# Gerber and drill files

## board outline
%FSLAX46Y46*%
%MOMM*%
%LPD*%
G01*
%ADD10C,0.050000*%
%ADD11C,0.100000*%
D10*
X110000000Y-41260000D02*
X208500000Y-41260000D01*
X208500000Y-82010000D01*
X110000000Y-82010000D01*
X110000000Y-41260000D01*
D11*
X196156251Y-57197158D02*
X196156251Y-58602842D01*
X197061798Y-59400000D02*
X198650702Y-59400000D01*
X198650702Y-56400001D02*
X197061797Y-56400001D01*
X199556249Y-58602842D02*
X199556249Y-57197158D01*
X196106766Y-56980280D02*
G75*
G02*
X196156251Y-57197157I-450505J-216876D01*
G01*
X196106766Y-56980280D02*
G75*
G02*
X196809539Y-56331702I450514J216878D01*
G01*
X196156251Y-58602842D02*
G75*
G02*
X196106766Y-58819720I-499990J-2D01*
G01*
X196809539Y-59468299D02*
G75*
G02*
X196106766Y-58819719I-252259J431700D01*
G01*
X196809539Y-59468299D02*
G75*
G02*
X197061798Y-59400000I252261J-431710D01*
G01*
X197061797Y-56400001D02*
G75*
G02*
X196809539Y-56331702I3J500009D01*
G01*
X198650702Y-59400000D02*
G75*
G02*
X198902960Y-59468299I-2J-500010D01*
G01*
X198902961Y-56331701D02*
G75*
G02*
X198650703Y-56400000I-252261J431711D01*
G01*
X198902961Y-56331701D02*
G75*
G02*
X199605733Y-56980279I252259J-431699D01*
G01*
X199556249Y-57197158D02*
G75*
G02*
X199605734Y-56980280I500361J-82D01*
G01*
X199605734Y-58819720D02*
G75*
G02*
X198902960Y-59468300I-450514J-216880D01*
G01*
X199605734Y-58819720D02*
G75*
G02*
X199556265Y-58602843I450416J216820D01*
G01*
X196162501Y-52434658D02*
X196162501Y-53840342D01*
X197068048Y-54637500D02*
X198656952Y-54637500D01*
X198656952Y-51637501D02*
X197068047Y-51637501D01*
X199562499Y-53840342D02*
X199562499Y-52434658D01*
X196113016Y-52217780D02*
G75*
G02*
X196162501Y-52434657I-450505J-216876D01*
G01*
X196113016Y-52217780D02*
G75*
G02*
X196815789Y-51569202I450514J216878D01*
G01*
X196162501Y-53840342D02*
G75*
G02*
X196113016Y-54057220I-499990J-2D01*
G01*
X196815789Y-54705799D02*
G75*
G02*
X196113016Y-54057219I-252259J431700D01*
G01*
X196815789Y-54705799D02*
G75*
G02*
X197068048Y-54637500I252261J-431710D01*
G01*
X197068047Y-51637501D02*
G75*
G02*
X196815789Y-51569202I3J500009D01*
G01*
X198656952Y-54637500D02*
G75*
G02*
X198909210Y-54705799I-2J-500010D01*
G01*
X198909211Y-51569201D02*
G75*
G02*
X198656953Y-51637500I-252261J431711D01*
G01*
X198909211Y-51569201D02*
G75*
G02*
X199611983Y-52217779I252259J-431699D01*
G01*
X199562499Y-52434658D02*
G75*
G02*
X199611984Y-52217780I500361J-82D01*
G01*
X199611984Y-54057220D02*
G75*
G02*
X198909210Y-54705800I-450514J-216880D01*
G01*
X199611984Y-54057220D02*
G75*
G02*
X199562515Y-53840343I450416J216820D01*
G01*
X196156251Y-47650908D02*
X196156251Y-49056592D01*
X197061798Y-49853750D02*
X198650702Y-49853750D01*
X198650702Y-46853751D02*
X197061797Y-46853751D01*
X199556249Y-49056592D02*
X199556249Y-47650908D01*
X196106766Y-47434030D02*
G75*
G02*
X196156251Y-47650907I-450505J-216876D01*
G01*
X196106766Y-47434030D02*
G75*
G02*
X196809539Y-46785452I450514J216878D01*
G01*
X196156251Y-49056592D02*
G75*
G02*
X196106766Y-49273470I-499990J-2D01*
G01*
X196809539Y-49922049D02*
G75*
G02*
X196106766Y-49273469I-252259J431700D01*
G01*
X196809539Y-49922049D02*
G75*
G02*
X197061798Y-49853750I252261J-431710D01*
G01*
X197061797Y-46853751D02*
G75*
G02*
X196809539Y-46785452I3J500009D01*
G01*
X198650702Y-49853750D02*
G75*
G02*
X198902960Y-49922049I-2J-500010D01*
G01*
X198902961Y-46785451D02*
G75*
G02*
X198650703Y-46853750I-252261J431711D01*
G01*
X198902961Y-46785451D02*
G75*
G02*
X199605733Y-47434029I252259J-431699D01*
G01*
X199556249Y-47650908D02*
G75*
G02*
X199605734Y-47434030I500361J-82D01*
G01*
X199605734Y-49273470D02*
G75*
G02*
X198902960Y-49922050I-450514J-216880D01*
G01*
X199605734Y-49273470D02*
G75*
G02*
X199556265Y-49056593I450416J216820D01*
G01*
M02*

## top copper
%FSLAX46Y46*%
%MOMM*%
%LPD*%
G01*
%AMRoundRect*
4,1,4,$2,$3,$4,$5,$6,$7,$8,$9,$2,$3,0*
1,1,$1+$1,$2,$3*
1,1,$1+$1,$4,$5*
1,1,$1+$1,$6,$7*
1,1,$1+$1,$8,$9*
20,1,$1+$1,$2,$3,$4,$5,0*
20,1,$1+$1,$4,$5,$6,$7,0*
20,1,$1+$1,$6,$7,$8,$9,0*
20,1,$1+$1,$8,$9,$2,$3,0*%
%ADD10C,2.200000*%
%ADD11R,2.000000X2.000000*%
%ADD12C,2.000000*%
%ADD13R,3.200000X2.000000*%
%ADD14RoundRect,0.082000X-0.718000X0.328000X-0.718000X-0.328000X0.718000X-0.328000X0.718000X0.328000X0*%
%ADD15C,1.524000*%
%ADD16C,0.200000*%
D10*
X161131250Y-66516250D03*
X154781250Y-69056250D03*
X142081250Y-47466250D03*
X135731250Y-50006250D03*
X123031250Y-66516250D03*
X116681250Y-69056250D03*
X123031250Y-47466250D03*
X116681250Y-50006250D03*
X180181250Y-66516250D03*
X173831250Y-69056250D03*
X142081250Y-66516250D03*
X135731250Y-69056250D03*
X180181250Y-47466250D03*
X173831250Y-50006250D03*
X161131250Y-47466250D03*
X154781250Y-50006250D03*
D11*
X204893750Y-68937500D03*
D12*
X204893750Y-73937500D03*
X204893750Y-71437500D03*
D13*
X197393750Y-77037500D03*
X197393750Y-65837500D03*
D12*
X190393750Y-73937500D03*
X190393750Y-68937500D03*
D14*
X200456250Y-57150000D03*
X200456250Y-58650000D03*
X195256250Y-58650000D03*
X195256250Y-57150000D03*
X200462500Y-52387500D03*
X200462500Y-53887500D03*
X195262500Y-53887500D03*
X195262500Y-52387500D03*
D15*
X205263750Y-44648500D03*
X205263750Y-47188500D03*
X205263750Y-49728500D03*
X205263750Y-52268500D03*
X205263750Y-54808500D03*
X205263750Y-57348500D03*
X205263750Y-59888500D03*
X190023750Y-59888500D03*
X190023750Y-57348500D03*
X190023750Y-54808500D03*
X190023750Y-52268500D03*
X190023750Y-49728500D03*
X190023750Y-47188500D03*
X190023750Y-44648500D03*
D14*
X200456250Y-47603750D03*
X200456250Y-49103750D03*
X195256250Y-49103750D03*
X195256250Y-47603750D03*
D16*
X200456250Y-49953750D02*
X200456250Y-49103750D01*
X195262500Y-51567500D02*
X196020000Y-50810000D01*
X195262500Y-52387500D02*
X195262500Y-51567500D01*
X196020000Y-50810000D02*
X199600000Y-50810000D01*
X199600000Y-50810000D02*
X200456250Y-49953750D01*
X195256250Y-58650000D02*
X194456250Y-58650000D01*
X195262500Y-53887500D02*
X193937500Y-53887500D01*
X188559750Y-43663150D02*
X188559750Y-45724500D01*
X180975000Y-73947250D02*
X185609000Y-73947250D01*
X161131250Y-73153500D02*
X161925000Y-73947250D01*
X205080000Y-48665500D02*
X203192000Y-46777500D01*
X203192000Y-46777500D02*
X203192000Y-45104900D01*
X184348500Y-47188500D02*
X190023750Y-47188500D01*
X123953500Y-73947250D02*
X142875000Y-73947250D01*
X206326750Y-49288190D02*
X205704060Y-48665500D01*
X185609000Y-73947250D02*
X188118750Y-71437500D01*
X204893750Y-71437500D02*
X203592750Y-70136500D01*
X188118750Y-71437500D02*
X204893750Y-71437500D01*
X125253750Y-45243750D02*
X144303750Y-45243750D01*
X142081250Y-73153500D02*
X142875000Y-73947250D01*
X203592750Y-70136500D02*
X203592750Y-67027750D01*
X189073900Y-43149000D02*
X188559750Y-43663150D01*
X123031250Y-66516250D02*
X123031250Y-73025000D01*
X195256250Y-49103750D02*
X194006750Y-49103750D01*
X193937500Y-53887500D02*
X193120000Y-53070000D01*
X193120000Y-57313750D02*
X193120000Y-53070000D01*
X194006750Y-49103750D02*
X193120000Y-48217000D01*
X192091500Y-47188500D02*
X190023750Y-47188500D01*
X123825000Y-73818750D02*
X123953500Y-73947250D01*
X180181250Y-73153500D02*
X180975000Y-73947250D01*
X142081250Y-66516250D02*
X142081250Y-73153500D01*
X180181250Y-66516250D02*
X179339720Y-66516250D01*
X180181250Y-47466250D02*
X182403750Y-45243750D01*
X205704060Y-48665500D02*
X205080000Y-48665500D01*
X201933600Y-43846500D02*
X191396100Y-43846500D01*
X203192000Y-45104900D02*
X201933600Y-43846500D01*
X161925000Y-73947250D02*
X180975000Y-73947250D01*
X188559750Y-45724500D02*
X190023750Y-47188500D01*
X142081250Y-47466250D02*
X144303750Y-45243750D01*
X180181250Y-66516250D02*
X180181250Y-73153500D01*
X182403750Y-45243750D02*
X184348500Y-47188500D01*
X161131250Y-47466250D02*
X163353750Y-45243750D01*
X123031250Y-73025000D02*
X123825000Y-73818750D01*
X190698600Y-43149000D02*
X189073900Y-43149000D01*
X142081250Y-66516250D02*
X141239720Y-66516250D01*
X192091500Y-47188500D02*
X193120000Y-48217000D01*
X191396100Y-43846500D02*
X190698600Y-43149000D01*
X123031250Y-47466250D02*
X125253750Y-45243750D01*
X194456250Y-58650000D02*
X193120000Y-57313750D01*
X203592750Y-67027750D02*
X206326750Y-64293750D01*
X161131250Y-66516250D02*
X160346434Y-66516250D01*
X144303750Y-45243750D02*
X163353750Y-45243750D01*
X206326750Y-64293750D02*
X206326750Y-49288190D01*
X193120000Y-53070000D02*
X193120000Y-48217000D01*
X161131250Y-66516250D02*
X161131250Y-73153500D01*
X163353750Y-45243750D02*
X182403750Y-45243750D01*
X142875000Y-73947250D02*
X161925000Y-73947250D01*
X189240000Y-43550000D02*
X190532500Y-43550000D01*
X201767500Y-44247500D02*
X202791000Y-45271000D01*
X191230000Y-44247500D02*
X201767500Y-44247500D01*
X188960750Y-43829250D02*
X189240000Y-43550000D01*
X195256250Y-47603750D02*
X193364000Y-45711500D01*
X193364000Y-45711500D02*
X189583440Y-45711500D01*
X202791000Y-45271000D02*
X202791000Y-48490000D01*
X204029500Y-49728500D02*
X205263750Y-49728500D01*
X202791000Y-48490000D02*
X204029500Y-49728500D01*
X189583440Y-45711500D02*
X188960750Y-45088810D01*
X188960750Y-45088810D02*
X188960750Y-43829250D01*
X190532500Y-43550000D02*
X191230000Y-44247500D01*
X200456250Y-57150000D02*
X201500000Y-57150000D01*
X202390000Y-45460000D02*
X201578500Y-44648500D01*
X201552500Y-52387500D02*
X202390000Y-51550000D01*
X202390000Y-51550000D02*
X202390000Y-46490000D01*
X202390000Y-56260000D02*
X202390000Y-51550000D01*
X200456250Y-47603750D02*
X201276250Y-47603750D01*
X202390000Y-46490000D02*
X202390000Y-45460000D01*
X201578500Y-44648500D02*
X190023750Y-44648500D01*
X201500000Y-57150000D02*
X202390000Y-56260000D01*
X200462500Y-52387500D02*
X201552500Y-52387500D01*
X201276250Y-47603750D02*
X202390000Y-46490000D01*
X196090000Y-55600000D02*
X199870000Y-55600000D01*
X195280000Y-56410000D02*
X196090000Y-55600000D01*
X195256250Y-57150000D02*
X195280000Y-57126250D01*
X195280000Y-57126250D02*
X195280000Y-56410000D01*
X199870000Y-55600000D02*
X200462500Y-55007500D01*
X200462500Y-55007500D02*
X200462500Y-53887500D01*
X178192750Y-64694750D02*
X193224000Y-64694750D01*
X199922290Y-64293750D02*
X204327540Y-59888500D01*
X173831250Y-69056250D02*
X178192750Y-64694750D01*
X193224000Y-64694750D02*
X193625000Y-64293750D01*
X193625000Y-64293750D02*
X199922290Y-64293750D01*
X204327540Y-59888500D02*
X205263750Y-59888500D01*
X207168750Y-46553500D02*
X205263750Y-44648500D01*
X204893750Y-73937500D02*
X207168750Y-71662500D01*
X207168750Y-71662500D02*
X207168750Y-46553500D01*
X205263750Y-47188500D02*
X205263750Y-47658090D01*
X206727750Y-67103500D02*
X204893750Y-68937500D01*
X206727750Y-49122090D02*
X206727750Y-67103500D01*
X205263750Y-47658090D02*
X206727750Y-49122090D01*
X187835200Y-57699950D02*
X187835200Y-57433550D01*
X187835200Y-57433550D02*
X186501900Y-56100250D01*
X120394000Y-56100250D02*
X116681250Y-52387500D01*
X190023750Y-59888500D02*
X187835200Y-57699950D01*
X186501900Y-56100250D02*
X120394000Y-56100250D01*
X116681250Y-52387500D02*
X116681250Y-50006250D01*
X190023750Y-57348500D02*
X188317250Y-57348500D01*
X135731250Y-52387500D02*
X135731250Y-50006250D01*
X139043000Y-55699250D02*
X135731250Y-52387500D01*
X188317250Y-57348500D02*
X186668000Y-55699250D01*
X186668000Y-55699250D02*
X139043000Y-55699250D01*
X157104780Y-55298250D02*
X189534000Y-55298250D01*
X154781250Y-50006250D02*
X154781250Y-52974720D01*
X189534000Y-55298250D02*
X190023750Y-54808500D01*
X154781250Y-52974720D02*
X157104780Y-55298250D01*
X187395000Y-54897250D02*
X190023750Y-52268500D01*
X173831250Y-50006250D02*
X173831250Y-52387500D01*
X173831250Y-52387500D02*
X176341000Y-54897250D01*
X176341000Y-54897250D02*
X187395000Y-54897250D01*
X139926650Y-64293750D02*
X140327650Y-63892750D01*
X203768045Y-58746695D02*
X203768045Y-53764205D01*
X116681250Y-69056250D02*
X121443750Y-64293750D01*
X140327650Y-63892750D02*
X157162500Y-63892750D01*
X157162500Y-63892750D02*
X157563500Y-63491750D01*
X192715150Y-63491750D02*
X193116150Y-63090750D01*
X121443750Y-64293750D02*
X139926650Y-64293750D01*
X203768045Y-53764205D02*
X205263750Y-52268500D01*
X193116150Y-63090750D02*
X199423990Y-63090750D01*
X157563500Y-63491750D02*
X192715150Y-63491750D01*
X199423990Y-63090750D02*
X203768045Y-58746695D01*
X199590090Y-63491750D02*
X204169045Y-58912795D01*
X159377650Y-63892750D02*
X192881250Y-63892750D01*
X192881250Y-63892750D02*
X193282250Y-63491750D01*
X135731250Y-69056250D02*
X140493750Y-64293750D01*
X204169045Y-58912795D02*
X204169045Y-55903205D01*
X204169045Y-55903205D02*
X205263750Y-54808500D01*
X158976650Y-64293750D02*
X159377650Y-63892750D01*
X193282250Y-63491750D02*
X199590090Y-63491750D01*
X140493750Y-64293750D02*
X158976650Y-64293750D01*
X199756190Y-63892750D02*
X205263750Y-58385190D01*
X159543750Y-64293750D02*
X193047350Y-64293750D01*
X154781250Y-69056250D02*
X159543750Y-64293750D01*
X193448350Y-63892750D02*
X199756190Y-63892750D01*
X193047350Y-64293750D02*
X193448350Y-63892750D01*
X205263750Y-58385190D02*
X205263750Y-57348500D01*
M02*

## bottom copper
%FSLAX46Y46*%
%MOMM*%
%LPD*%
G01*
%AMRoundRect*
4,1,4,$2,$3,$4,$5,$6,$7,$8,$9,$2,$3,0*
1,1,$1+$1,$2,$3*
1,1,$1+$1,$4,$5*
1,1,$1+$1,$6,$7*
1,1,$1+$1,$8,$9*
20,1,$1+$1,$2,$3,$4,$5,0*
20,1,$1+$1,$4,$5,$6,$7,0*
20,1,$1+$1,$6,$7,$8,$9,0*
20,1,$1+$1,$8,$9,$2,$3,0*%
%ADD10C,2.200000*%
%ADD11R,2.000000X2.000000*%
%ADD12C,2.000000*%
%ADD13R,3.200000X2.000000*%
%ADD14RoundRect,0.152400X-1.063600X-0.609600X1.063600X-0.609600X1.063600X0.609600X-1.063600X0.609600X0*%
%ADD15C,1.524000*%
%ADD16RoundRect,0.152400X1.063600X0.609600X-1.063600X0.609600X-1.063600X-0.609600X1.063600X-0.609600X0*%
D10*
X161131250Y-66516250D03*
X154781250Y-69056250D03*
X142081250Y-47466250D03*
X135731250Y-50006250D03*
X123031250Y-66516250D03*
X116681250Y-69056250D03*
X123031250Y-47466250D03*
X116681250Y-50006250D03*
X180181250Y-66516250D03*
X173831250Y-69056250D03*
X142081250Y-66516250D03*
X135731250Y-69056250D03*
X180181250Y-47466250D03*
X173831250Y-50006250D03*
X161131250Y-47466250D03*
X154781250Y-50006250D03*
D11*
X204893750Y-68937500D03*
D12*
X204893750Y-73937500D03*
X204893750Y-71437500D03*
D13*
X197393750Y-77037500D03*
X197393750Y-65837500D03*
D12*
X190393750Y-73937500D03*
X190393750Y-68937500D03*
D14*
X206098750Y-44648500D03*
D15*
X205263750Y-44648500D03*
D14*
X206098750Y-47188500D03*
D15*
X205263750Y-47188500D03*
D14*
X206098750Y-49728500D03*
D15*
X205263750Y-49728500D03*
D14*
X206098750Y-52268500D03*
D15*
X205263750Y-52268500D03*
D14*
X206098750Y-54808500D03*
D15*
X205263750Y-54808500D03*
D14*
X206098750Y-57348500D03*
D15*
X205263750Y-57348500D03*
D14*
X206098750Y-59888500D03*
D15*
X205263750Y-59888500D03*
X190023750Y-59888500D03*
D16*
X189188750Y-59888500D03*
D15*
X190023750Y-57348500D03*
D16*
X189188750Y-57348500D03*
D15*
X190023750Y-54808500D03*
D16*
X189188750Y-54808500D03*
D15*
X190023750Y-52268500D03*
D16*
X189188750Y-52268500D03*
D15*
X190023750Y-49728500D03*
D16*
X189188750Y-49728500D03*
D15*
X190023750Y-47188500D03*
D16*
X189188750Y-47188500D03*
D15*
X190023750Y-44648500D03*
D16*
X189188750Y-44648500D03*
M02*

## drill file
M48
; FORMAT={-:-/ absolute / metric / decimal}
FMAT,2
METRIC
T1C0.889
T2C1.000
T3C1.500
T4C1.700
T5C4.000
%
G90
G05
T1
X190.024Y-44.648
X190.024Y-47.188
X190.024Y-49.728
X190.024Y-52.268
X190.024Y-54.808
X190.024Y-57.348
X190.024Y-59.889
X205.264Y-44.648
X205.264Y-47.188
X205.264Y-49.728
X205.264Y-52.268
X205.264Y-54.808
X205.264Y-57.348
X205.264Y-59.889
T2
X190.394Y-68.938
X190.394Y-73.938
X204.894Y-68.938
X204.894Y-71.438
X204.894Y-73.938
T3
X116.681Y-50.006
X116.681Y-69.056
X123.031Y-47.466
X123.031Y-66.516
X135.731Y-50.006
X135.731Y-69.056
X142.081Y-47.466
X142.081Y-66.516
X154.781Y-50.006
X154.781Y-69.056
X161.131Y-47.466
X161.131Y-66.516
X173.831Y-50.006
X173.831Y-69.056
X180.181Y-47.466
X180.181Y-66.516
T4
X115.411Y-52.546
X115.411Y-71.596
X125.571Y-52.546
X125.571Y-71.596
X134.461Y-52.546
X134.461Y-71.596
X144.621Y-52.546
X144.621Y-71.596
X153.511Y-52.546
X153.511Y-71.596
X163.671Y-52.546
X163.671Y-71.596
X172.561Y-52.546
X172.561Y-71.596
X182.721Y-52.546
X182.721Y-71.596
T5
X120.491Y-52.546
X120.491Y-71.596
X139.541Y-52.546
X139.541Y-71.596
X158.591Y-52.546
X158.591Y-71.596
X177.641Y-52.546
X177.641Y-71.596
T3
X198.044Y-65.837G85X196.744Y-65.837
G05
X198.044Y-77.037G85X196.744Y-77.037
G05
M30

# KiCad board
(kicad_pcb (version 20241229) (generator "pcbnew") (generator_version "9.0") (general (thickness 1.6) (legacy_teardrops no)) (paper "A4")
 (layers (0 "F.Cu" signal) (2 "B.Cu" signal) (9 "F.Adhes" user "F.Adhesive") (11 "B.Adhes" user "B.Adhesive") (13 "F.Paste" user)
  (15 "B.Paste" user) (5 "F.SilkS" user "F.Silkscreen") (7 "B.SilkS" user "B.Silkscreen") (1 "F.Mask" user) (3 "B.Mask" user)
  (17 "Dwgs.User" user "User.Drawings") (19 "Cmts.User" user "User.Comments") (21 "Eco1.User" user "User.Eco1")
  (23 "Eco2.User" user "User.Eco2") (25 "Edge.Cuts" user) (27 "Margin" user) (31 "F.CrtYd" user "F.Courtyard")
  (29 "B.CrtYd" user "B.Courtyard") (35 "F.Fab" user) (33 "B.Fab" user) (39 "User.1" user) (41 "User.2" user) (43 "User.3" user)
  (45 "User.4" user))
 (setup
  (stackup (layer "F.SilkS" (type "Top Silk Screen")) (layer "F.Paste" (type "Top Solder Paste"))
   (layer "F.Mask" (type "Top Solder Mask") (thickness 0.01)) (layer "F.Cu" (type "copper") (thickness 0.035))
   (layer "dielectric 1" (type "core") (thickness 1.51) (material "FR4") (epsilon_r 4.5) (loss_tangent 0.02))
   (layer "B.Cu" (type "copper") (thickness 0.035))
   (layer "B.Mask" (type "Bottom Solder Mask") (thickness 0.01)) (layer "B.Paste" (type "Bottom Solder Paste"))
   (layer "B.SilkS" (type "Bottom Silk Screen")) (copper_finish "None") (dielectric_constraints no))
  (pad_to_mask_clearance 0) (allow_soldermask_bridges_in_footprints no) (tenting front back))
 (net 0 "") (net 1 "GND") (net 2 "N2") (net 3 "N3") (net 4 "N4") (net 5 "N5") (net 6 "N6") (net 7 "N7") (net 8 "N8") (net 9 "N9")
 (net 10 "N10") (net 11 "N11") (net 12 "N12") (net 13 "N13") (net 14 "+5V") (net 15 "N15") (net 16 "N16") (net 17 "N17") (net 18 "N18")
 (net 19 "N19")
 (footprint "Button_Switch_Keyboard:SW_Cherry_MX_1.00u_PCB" (layer "F.Cu") (at 161.13125 66.51625)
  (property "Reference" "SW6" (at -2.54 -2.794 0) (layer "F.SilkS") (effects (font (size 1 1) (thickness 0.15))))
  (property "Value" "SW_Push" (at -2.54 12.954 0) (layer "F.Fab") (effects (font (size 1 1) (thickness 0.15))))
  (pad "" np_thru_hole circle (at -7.62 5.08) (size 1.7 1.7) (drill 1.7) (layers "*.Cu" "*.Mask"))
  (pad "" np_thru_hole circle (at -2.54 5.08) (size 4 4) (drill 4) (layers "*.Cu" "*.Mask"))
  (pad "" np_thru_hole circle (at 2.54 5.08) (size 1.7 1.7) (drill 1.7) (layers "*.Cu" "*.Mask"))
  (pad "1" thru_hole circle (at 0 0) (size 2.2 2.2) (drill 1.5) (layers "*.Cu" "*.Mask") (remove_unused_layers no) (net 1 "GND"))
  (pad "2" thru_hole circle (at -6.35 2.54) (size 2.2 2.2) (drill 1.5) (layers "*.Cu" "*.Mask") (remove_unused_layers no) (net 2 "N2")))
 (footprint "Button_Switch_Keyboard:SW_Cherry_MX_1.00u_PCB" (layer "F.Cu") (at 142.08125 47.46625)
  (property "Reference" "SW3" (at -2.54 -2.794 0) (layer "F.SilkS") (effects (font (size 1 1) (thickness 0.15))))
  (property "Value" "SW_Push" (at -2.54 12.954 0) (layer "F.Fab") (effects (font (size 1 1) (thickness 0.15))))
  (pad "" np_thru_hole circle (at -7.62 5.08) (size 1.7 1.7) (drill 1.7) (layers "*.Cu" "*.Mask"))
  (pad "" np_thru_hole circle (at -2.54 5.08) (size 4 4) (drill 4) (layers "*.Cu" "*.Mask"))
  (pad "" np_thru_hole circle (at 2.54 5.08) (size 1.7 1.7) (drill 1.7) (layers "*.Cu" "*.Mask"))
  (pad "1" thru_hole circle (at 0 0) (size 2.2 2.2) (drill 1.5) (layers "*.Cu" "*.Mask") (remove_unused_layers no) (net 1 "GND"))
  (pad "2" thru_hole circle (at -6.35 2.54) (size 2.2 2.2) (drill 1.5) (layers "*.Cu" "*.Mask") (remove_unused_layers no) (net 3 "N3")))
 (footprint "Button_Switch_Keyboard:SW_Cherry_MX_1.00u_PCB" (layer "F.Cu") (at 123.03125 66.51625)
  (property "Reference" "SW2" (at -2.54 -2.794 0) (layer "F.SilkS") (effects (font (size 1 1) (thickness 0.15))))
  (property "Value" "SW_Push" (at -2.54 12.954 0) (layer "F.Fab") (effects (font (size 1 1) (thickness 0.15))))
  (pad "" np_thru_hole circle (at -7.62 5.08) (size 1.7 1.7) (drill 1.7) (layers "*.Cu" "*.Mask"))
  (pad "" np_thru_hole circle (at -2.54 5.08) (size 4 4) (drill 4) (layers "*.Cu" "*.Mask"))
  (pad "" np_thru_hole circle (at 2.54 5.08) (size 1.7 1.7) (drill 1.7) (layers "*.Cu" "*.Mask"))
  (pad "1" thru_hole circle (at 0 0) (size 2.2 2.2) (drill 1.5) (layers "*.Cu" "*.Mask") (remove_unused_layers no) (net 1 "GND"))
  (pad "2" thru_hole circle (at -6.35 2.54) (size 2.2 2.2) (drill 1.5) (layers "*.Cu" "*.Mask") (remove_unused_layers no) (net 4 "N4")))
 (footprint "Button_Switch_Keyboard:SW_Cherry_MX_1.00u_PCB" (layer "F.Cu") (at 123.03125 47.46625)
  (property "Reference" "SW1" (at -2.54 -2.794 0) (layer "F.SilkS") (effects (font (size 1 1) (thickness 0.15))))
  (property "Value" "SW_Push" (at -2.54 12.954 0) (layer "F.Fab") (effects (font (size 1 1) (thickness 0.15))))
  (pad "" np_thru_hole circle (at -7.62 5.08) (size 1.7 1.7) (drill 1.7) (layers "*.Cu" "*.Mask"))
  (pad "" np_thru_hole circle (at -2.54 5.08) (size 4 4) (drill 4) (layers "*.Cu" "*.Mask"))
  (pad "" np_thru_hole circle (at 2.54 5.08) (size 1.7 1.7) (drill 1.7) (layers "*.Cu" "*.Mask"))
  (pad "1" thru_hole circle (at 0 0) (size 2.2 2.2) (drill 1.5) (layers "*.Cu" "*.Mask") (remove_unused_layers no) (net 1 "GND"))
  (pad "2" thru_hole circle (at -6.35 2.54) (size 2.2 2.2) (drill 1.5) (layers "*.Cu" "*.Mask") (remove_unused_layers no) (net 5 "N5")))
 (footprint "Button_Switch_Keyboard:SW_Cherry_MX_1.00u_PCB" (layer "F.Cu") (at 180.18125 66.51625)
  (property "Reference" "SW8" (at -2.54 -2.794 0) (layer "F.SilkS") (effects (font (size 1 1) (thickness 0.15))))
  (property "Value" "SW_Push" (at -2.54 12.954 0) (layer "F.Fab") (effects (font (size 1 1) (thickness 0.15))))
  (pad "" np_thru_hole circle (at -7.62 5.08) (size 1.7 1.7) (drill 1.7) (layers "*.Cu" "*.Mask"))
  (pad "" np_thru_hole circle (at -2.54 5.08) (size 4 4) (drill 4) (layers "*.Cu" "*.Mask"))
  (pad "" np_thru_hole circle (at 2.54 5.08) (size 1.7 1.7) (drill 1.7) (layers "*.Cu" "*.Mask"))
  (pad "1" thru_hole circle (at 0 0) (size 2.2 2.2) (drill 1.5) (layers "*.Cu" "*.Mask") (remove_unused_layers no) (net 1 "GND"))
  (pad "2" thru_hole circle (at -6.35 2.54) (size 2.2 2.2) (drill 1.5) (layers "*.Cu" "*.Mask") (remove_unused_layers no) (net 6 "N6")))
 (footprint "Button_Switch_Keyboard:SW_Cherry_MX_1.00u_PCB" (layer "F.Cu") (at 142.08125 66.51625)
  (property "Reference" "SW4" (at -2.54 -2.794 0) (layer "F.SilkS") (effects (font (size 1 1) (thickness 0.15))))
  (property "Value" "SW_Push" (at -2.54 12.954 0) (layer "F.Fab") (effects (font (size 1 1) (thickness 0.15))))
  (pad "" np_thru_hole circle (at -7.62 5.08) (size 1.7 1.7) (drill 1.7) (layers "*.Cu" "*.Mask"))
  (pad "" np_thru_hole circle (at -2.54 5.08) (size 4 4) (drill 4) (layers "*.Cu" "*.Mask"))
  (pad "" np_thru_hole circle (at 2.54 5.08) (size 1.7 1.7) (drill 1.7) (layers "*.Cu" "*.Mask"))
  (pad "1" thru_hole circle (at 0 0) (size 2.2 2.2) (drill 1.5) (layers "*.Cu" "*.Mask") (remove_unused_layers no) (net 1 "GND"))
  (pad "2" thru_hole circle (at -6.35 2.54) (size 2.2 2.2) (drill 1.5) (layers "*.Cu" "*.Mask") (remove_unused_layers no) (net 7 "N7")))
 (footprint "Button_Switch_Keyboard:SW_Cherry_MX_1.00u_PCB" (layer "F.Cu") (at 180.18125 47.46625)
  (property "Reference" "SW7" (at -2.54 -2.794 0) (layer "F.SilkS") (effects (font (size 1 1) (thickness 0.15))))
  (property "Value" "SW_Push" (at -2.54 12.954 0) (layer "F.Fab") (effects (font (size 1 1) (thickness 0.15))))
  (pad "" np_thru_hole circle (at -7.62 5.08) (size 1.7 1.7) (drill 1.7) (layers "*.Cu" "*.Mask"))
  (pad "" np_thru_hole circle (at -2.54 5.08) (size 4 4) (drill 4) (layers "*.Cu" "*.Mask"))
  (pad "" np_thru_hole circle (at 2.54 5.08) (size 1.7 1.7) (drill 1.7) (layers "*.Cu" "*.Mask"))
  (pad "1" thru_hole circle (at 0 0) (size 2.2 2.2) (drill 1.5) (layers "*.Cu" "*.Mask") (remove_unused_layers no) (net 1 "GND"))
  (pad "2" thru_hole circle (at -6.35 2.54) (size 2.2 2.2) (drill 1.5) (layers "*.Cu" "*.Mask") (remove_unused_layers no) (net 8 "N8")))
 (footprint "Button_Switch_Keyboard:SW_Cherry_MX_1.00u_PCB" (layer "F.Cu") (at 161.13125 47.46625)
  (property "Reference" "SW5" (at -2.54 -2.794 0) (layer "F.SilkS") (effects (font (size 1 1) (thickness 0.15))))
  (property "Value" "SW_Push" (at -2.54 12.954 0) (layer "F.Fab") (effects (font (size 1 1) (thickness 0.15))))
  (pad "" np_thru_hole circle (at -7.62 5.08) (size 1.7 1.7) (drill 1.7) (layers "*.Cu" "*.Mask"))
  (pad "" np_thru_hole circle (at -2.54 5.08) (size 4 4) (drill 4) (layers "*.Cu" "*.Mask"))
  (pad "" np_thru_hole circle (at 2.54 5.08) (size 1.7 1.7) (drill 1.7) (layers "*.Cu" "*.Mask"))
  (pad "1" thru_hole circle (at 0 0) (size 2.2 2.2) (drill 1.5) (layers "*.Cu" "*.Mask") (remove_unused_layers no) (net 1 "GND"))
  (pad "2" thru_hole circle (at -6.35 2.54) (size 2.2 2.2) (drill 1.5) (layers "*.Cu" "*.Mask") (remove_unused_layers no) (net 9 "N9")))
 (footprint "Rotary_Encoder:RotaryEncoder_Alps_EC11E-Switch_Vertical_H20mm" (layer "B.Cu") (at 204.89375 68.9375 180)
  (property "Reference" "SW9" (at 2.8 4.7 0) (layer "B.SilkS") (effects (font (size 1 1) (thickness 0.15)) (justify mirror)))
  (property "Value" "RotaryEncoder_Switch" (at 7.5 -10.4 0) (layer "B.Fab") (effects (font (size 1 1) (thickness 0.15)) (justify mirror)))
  (pad "A" thru_hole rect (at 0 0 180) (size 2 2) (drill 1) (layers "*.Cu" "*.Mask") (remove_unused_layers no) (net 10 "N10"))
  (pad "B" thru_hole circle (at 0 -5 180) (size 2 2) (drill 1) (layers "*.Cu" "*.Mask") (remove_unused_layers no) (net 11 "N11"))
  (pad "C" thru_hole circle (at 0 -2.5 180) (size 2 2) (drill 1) (layers "*.Cu" "*.Mask") (remove_unused_layers no) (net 1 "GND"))
  (pad "MP" thru_hole rect (at 7.5 -8.1 180) (size 3.2 2) (drill oval 2.8 1.5) (layers "*.Cu" "*.Mask") (remove_unused_layers no))
  (pad "MP" thru_hole rect (at 7.5 3.1 180) (size 3.2 2) (drill oval 2.8 1.5) (layers "*.Cu" "*.Mask") (remove_unused_layers no))
  (pad "S1" thru_hole circle (at 14.5 -5 180) (size 2 2) (drill 1) (layers "*.Cu" "*.Mask") (remove_unused_layers no) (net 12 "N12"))
  (pad "S2" thru_hole circle (at 14.5 0 180) (size 2 2) (drill 1) (layers "*.Cu" "*.Mask") (remove_unused_layers no) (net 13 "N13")))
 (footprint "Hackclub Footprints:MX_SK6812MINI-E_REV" (layer "B.Cu") (at 197.85625 62.98)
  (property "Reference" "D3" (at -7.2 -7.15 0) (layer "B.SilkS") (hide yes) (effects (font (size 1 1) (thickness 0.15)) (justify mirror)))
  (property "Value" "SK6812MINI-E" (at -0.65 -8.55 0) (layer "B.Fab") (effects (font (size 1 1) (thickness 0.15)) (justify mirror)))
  (fp_line (start -1.699999 -5.782842) (end -1.699999 -4.377158) (stroke (width 0.1) (type solid)) (layer "Edge.Cuts"))
  (fp_line (start -0.794452 -3.58) (end 0.794452 -3.58) (stroke (width 0.1) (type solid)) (layer "Edge.Cuts"))
  (fp_line (start 0.794452 -6.579999) (end -0.794453 -6.579999) (stroke (width 0.1) (type solid)) (layer "Edge.Cuts"))
  (fp_line (start 1.699999 -4.377158) (end 1.699999 -5.782842) (stroke (width 0.1) (type solid)) (layer "Edge.Cuts"))
  (fp_arc (start -1.749484 -5.99972) (mid -1.712527 -5.894068) (end -1.699999 -5.782843) (stroke (width 0.1) (type solid))
   (layer "Edge.Cuts"))
  (fp_arc (start -1.749484 -5.99972) (mid -1.638071 -6.584035) (end -1.046711 -6.648298) (stroke (width 0.1) (type solid))
   (layer "Edge.Cuts"))
  (fp_arc (start -1.699999 -4.377158) (mid -1.712527 -4.265932) (end -1.749484 -4.16028) (stroke (width 0.1) (type solid))
   (layer "Edge.Cuts"))
  (fp_arc (start -1.046711 -3.511701) (mid -1.638072 -3.575965) (end -1.749484 -4.160281) (stroke (width 0.1) (type solid))
   (layer "Edge.Cuts"))
  (fp_arc (start -1.046711 -3.511701) (mid -0.925123 -3.562623) (end -0.794452 -3.58) (stroke (width 0.1) (type solid)) (layer "Edge.Cuts"))
  (fp_arc (start -0.794453 -6.579999) (mid -0.925123 -6.597376) (end -1.046711 -6.648298) (stroke (width 0.1) (type solid))
   (layer "Edge.Cuts"))
  (fp_arc (start 0.794452 -3.58) (mid 0.925122 -3.562623) (end 1.04671 -3.511701) (stroke (width 0.1) (type solid)) (layer "Edge.Cuts"))
  (fp_arc (start 1.046711 -6.648299) (mid 0.925123 -6.597377) (end 0.794453 -6.58) (stroke (width 0.1) (type solid)) (layer "Edge.Cuts"))
  (fp_arc (start 1.046711 -6.648299) (mid 1.638071 -6.584036) (end 1.749484 -5.99972) (stroke (width 0.1) (type solid)) (layer "Edge.Cuts"))
  (fp_arc (start 1.699999 -5.782842) (mid 1.712536 -5.894065) (end 1.749484 -5.99972) (stroke (width 0.1) (type solid)) (layer "Edge.Cuts"))
  (fp_arc (start 1.749484 -4.16028) (mid 1.638072 -3.575963) (end 1.046711 -3.511703) (stroke (width 0.1) (type solid)) (layer "Edge.Cuts"))
  (fp_arc (start 1.749484 -4.16028) (mid 1.712526 -4.265931) (end 1.699999 -4.377157) (stroke (width 0.1) (type solid)) (layer "Edge.Cuts"))
  (pad "1" smd roundrect (at 2.6 -5.83 270) (size 0.82 1.6) (layers "F.Cu" "F.Mask" "F.Paste") (roundrect_rratio 0.1) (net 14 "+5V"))
  (pad "2" smd roundrect (at 2.6 -4.33 270) (size 0.82 1.6) (layers "F.Cu" "F.Mask" "F.Paste") (roundrect_rratio 0.1) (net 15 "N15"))
  (pad "3" smd roundrect (at -2.6 -4.33 270) (size 0.82 1.6) (layers "F.Cu" "F.Mask" "F.Paste") (roundrect_rratio 0.1) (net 1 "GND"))
  (pad "4" smd roundrect (at -2.6 -5.83 270) (size 0.82 1.6) (layers "F.Cu" "F.Mask" "F.Paste") (roundrect_rratio 0.1) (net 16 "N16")))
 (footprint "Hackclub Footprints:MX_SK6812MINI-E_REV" (layer "B.Cu") (at 197.8625 58.2175)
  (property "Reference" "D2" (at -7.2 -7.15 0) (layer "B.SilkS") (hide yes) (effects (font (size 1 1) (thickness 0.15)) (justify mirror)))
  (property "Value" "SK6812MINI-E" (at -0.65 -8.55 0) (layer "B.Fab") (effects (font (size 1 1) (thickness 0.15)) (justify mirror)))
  (fp_line (start -1.699999 -5.782842) (end -1.699999 -4.377158) (stroke (width 0.1) (type solid)) (layer "Edge.Cuts"))
  (fp_line (start -0.794452 -3.58) (end 0.794452 -3.58) (stroke (width 0.1) (type solid)) (layer "Edge.Cuts"))
  (fp_line (start 0.794452 -6.579999) (end -0.794453 -6.579999) (stroke (width 0.1) (type solid)) (layer "Edge.Cuts"))
  (fp_line (start 1.699999 -4.377158) (end 1.699999 -5.782842) (stroke (width 0.1) (type solid)) (layer "Edge.Cuts"))
  (fp_arc (start -1.749484 -5.99972) (mid -1.712527 -5.894068) (end -1.699999 -5.782843) (stroke (width 0.1) (type solid))
   (layer "Edge.Cuts"))
  (fp_arc (start -1.749484 -5.99972) (mid -1.638071 -6.584035) (end -1.046711 -6.648298) (stroke (width 0.1) (type solid))
   (layer "Edge.Cuts"))
  (fp_arc (start -1.699999 -4.377158) (mid -1.712527 -4.265932) (end -1.749484 -4.16028) (stroke (width 0.1) (type solid))
   (layer "Edge.Cuts"))
  (fp_arc (start -1.046711 -3.511701) (mid -1.638072 -3.575965) (end -1.749484 -4.160281) (stroke (width 0.1) (type solid))
   (layer "Edge.Cuts"))
  (fp_arc (start -1.046711 -3.511701) (mid -0.925123 -3.562623) (end -0.794452 -3.58) (stroke (width 0.1) (type solid)) (layer "Edge.Cuts"))
  (fp_arc (start -0.794453 -6.579999) (mid -0.925123 -6.597376) (end -1.046711 -6.648298) (stroke (width 0.1) (type solid))
   (layer "Edge.Cuts"))
  (fp_arc (start 0.794452 -3.58) (mid 0.925122 -3.562623) (end 1.04671 -3.511701) (stroke (width 0.1) (type solid)) (layer "Edge.Cuts"))
  (fp_arc (start 1.046711 -6.648299) (mid 0.925123 -6.597377) (end 0.794453 -6.58) (stroke (width 0.1) (type solid)) (layer "Edge.Cuts"))
  (fp_arc (start 1.046711 -6.648299) (mid 1.638071 -6.584036) (end 1.749484 -5.99972) (stroke (width 0.1) (type solid)) (layer "Edge.Cuts"))
  (fp_arc (start 1.699999 -5.782842) (mid 1.712536 -5.894065) (end 1.749484 -5.99972) (stroke (width 0.1) (type solid)) (layer "Edge.Cuts"))
  (fp_arc (start 1.749484 -4.16028) (mid 1.638072 -3.575963) (end 1.046711 -3.511703) (stroke (width 0.1) (type solid)) (layer "Edge.Cuts"))
  (fp_arc (start 1.749484 -4.16028) (mid 1.712526 -4.265931) (end 1.699999 -4.377157) (stroke (width 0.1) (type solid)) (layer "Edge.Cuts"))
  (pad "1" smd roundrect (at 2.6 -5.83 270) (size 0.82 1.6) (layers "F.Cu" "F.Mask" "F.Paste") (roundrect_rratio 0.1) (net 14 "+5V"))
  (pad "2" smd roundrect (at 2.6 -4.33 270) (size 0.82 1.6) (layers "F.Cu" "F.Mask" "F.Paste") (roundrect_rratio 0.1) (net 16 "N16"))
  (pad "3" smd roundrect (at -2.6 -4.33 270) (size 0.82 1.6) (layers "F.Cu" "F.Mask" "F.Paste") (roundrect_rratio 0.1) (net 1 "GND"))
  (pad "4" smd roundrect (at -2.6 -5.83 270) (size 0.82 1.6) (layers "F.Cu" "F.Mask" "F.Paste") (roundrect_rratio 0.1) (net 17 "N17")))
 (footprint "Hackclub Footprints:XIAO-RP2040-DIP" (layer "B.Cu") (at 197.64375 52.2685 180)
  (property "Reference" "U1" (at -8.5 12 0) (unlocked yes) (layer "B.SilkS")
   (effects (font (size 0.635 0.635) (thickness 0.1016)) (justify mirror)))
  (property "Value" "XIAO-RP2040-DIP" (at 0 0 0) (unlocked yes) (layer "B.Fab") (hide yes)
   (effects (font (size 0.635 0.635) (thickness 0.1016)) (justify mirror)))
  (pad "1" smd roundrect (at -8.455 7.62) (size 2.432 1.524) (layers "B.Cu" "B.Mask") (roundrect_rratio 0.1) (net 11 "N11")
   (thermal_bridge_angle 45))
  (pad "1" thru_hole circle (at -7.62 7.62) (size 1.524 1.524) (drill 0.889) (layers "*.Cu" "*.Mask") (remove_unused_layers no)
   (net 11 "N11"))
  (pad "2" smd roundrect (at -8.455 5.08) (size 2.432 1.524) (layers "B.Cu" "B.Mask") (roundrect_rratio 0.1) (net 10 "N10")
   (thermal_bridge_angle 45))
  (pad "2" thru_hole circle (at -7.62 5.08) (size 1.524 1.524) (drill 0.889) (layers "*.Cu" "*.Mask") (remove_unused_layers no)
   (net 10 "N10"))
  (pad "3" smd roundrect (at -8.455 2.54) (size 2.432 1.524) (layers "B.Cu" "B.Mask") (roundrect_rratio 0.1) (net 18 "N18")
   (thermal_bridge_angle 45))
  (pad "3" thru_hole circle (at -7.62 2.54) (size 1.524 1.524) (drill 0.889) (layers "*.Cu" "*.Mask") (remove_unused_layers no)
   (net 18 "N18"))
  (pad "4" smd roundrect (at -8.455 0) (size 2.432 1.524) (layers "B.Cu" "B.Mask") (roundrect_rratio 0.1) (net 4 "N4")
   (thermal_bridge_angle 45))
  (pad "4" thru_hole circle (at -7.62 0) (size 1.524 1.524) (drill 0.889) (layers "*.Cu" "*.Mask") (remove_unused_layers no) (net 4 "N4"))
  (pad "5" smd roundrect (at -8.455 -2.54) (size 2.432 1.524) (layers "B.Cu" "B.Mask") (roundrect_rratio 0.1) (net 7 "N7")
   (thermal_bridge_angle 45))
  (pad "5" thru_hole circle (at -7.62 -2.54) (size 1.524 1.524) (drill 0.889) (layers "*.Cu" "*.Mask") (remove_unused_layers no)
   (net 7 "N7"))
  (pad "6" smd roundrect (at -8.455 -5.08) (size 2.432 1.524) (layers "B.Cu" "B.Mask") (roundrect_rratio 0.1) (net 2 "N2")
   (thermal_bridge_angle 45))
  (pad "6" thru_hole circle (at -7.62 -5.08) (size 1.524 1.524) (drill 0.889) (layers "*.Cu" "*.Mask") (remove_unused_layers no)
   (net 2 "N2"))
  (pad "7" smd roundrect (at -8.455 -7.62) (size 2.432 1.524) (layers "B.Cu" "B.Mask") (roundrect_rratio 0.1) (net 6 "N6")
   (thermal_bridge_angle 45))
  (pad "7" thru_hole circle (at -7.62 -7.62) (size 1.524 1.524) (drill 0.889) (layers "*.Cu" "*.Mask") (remove_unused_layers no)
   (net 6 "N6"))
  (pad "8" thru_hole circle (at 7.62 -7.62 180) (size 1.524 1.524) (drill 0.889) (layers "*.Cu" "*.Mask") (remove_unused_layers no)
   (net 5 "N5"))
  (pad "8" smd roundrect (at 8.455 -7.62 180) (size 2.432 1.524) (layers "B.Cu" "B.Mask") (roundrect_rratio 0.1) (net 5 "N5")
   (thermal_bridge_angle 45))
  (pad "9" thru_hole circle (at 7.62 -5.08 180) (size 1.524 1.524) (drill 0.889) (layers "*.Cu" "*.Mask") (remove_unused_layers no)
   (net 3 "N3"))
  (pad "9" smd roundrect (at 8.455 -5.08 180) (size 2.432 1.524) (layers "B.Cu" "B.Mask") (roundrect_rratio 0.1) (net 3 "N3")
   (thermal_bridge_angle 45))
  (pad "10" thru_hole circle (at 7.62 -2.54 180) (size 1.524 1.524) (drill 0.889) (layers "*.Cu" "*.Mask") (remove_unused_layers no)
   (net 9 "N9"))
  (pad "10" smd roundrect (at 8.455 -2.54 180) (size 2.432 1.524) (layers "B.Cu" "B.Mask") (roundrect_rratio 0.1) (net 9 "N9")
   (thermal_bridge_angle 45))
  (pad "11" thru_hole circle (at 7.62 0 180) (size 1.524 1.524) (drill 0.889) (layers "*.Cu" "*.Mask") (remove_unused_layers no)
   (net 8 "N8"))
  (pad "11" smd roundrect (at 8.455 0 180) (size 2.432 1.524) (layers "B.Cu" "B.Mask") (roundrect_rratio 0.1) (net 8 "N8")
   (thermal_bridge_angle 45))
  (pad "12" thru_hole circle (at 7.62 2.54 180) (size 1.524 1.524) (drill 0.889) (layers "*.Cu" "*.Mask") (remove_unused_layers no)
   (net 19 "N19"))
  (pad "12" smd roundrect (at 8.455 2.54 180) (size 2.432 1.524) (layers "B.Cu" "B.Mask") (roundrect_rratio 0.1) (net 19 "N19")
   (thermal_bridge_angle 45))
  (pad "13" thru_hole circle (at 7.62 5.08 180) (size 1.524 1.524) (drill 0.889) (layers "*.Cu" "*.Mask") (remove_unused_layers no)
   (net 1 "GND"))
  (pad "13" smd roundrect (at 8.455 5.08 180) (size 2.432 1.524) (layers "B.Cu" "B.Mask") (roundrect_rratio 0.1) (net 1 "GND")
   (thermal_bridge_angle 45))
  (pad "14" thru_hole circle (at 7.62 7.62 180) (size 1.524 1.524) (drill 0.889) (layers "*.Cu" "*.Mask") (remove_unused_layers no)
   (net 14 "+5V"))
  (pad "14" smd roundrect (at 8.455 7.62 180) (size 2.432 1.524) (layers "B.Cu" "B.Mask") (roundrect_rratio 0.1) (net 14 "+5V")
   (thermal_bridge_angle 45)))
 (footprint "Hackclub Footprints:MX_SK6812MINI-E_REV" (layer "B.Cu") (at 197.85625 53.43375)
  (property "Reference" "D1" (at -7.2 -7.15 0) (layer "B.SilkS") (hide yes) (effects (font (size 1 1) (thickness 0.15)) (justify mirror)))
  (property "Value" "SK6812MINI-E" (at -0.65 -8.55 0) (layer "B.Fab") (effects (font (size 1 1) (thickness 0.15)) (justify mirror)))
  (fp_line (start -1.699999 -5.782842) (end -1.699999 -4.377158) (stroke (width 0.1) (type solid)) (layer "Edge.Cuts"))
  (fp_line (start -0.794452 -3.58) (end 0.794452 -3.58) (stroke (width 0.1) (type solid)) (layer "Edge.Cuts"))
  (fp_line (start 0.794452 -6.579999) (end -0.794453 -6.579999) (stroke (width 0.1) (type solid)) (layer "Edge.Cuts"))
  (fp_line (start 1.699999 -4.377158) (end 1.699999 -5.782842) (stroke (width 0.1) (type solid)) (layer "Edge.Cuts"))
  (fp_arc (start -1.749484 -5.99972) (mid -1.712527 -5.894068) (end -1.699999 -5.782843) (stroke (width 0.1) (type solid))
   (layer "Edge.Cuts"))
  (fp_arc (start -1.749484 -5.99972) (mid -1.638071 -6.584035) (end -1.046711 -6.648298) (stroke (width 0.1) (type solid))
   (layer "Edge.Cuts"))
  (fp_arc (start -1.699999 -4.377158) (mid -1.712527 -4.265932) (end -1.749484 -4.16028) (stroke (width 0.1) (type solid))
   (layer "Edge.Cuts"))
  (fp_arc (start -1.046711 -3.511701) (mid -1.638072 -3.575965) (end -1.749484 -4.160281) (stroke (width 0.1) (type solid))
   (layer "Edge.Cuts"))
  (fp_arc (start -1.046711 -3.511701) (mid -0.925123 -3.562623) (end -0.794452 -3.58) (stroke (width 0.1) (type solid)) (layer "Edge.Cuts"))
  (fp_arc (start -0.794453 -6.579999) (mid -0.925123 -6.597376) (end -1.046711 -6.648298) (stroke (width 0.1) (type solid))
   (layer "Edge.Cuts"))
  (fp_arc (start 0.794452 -3.58) (mid 0.925122 -3.562623) (end 1.04671 -3.511701) (stroke (width 0.1) (type solid)) (layer "Edge.Cuts"))
  (fp_arc (start 1.046711 -6.648299) (mid 0.925123 -6.597377) (end 0.794453 -6.58) (stroke (width 0.1) (type solid)) (layer "Edge.Cuts"))
  (fp_arc (start 1.046711 -6.648299) (mid 1.638071 -6.584036) (end 1.749484 -5.99972) (stroke (width 0.1) (type solid)) (layer "Edge.Cuts"))
  (fp_arc (start 1.699999 -5.782842) (mid 1.712536 -5.894065) (end 1.749484 -5.99972) (stroke (width 0.1) (type solid)) (layer "Edge.Cuts"))
  (fp_arc (start 1.749484 -4.16028) (mid 1.638072 -3.575963) (end 1.046711 -3.511703) (stroke (width 0.1) (type solid)) (layer "Edge.Cuts"))
  (fp_arc (start 1.749484 -4.16028) (mid 1.712526 -4.265931) (end 1.699999 -4.377157) (stroke (width 0.1) (type solid)) (layer "Edge.Cuts"))
  (pad "1" smd roundrect (at 2.6 -5.83 270) (size 0.82 1.6) (layers "F.Cu" "F.Mask" "F.Paste") (roundrect_rratio 0.1) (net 14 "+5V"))
  (pad "2" smd roundrect (at 2.6 -4.33 270) (size 0.82 1.6) (layers "F.Cu" "F.Mask" "F.Paste") (roundrect_rratio 0.1) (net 17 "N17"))
  (pad "3" smd roundrect (at -2.6 -4.33 270) (size 0.82 1.6) (layers "F.Cu" "F.Mask" "F.Paste") (roundrect_rratio 0.1) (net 1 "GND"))
  (pad "4" smd roundrect (at -2.6 -5.83 270) (size 0.82 1.6) (layers "F.Cu" "F.Mask" "F.Paste") (roundrect_rratio 0.1) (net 18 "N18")))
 (gr_rect (start 110 41.26) (end 208.5 82.01) (stroke (width 0.05) (type default)) (fill no) (layer "Edge.Cuts"))
 (segment (start 200.45625 49.95375) (end 200.45625 49.10375) (width 0.2) (layer "F.Cu") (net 17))
 (segment (start 195.2625 51.5675) (end 196.02 50.81) (width 0.2) (layer "F.Cu") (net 17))
 (segment (start 195.2625 52.3875) (end 195.2625 51.5675) (width 0.2) (layer "F.Cu") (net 17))
 (segment (start 196.02 50.81) (end 199.6 50.81) (width 0.2) (layer "F.Cu") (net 17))
 (segment (start 199.6 50.81) (end 200.45625 49.95375) (width 0.2) (layer "F.Cu") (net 17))
 (segment (start 195.25625 58.65) (end 194.45625 58.65) (width 0.2) (layer "F.Cu") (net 1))
 (segment (start 195.2625 53.8875) (end 193.9375 53.8875) (width 0.2) (layer "F.Cu") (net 1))
 (segment (start 188.55975 43.66315) (end 188.55975 45.7245) (width 0.2) (layer "F.Cu") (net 1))
 (segment (start 180.975 73.94725) (end 185.609 73.94725) (width 0.2) (layer "F.Cu") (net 1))
 (segment (start 161.13125 73.1535) (end 161.925 73.94725) (width 0.2) (layer "F.Cu") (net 1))
 (segment (start 205.08 48.6655) (end 203.192 46.7775) (width 0.2) (layer "F.Cu") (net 1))
 (segment (start 203.192 46.7775) (end 203.192 45.1049) (width 0.2) (layer "F.Cu") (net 1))
 (segment (start 184.3485 47.1885) (end 190.02375 47.1885) (width 0.2) (layer "F.Cu") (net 1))
 (segment (start 123.9535 73.94725) (end 142.875 73.94725) (width 0.2) (layer "F.Cu") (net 1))
 (segment (start 206.32675 49.28819) (end 205.70406 48.6655) (width 0.2) (layer "F.Cu") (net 1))
 (segment (start 185.609 73.94725) (end 188.11875 71.4375) (width 0.2) (layer "F.Cu") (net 1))
 (segment (start 204.89375 71.4375) (end 203.59275 70.1365) (width 0.2) (layer "F.Cu") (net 1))
 (segment (start 188.11875 71.4375) (end 204.89375 71.4375) (width 0.2) (layer "F.Cu") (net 1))
 (segment (start 125.25375 45.24375) (end 144.30375 45.24375) (width 0.2) (layer "F.Cu") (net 1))
 (segment (start 142.08125 73.1535) (end 142.875 73.94725) (width 0.2) (layer "F.Cu") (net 1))
 (segment (start 203.59275 70.1365) (end 203.59275 67.02775) (width 0.2) (layer "F.Cu") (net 1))
 (segment (start 189.0739 43.149) (end 188.55975 43.66315) (width 0.2) (layer "F.Cu") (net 1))
 (segment (start 123.03125 66.51625) (end 123.03125 73.025) (width 0.2) (layer "F.Cu") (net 1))
 (segment (start 195.25625 49.10375) (end 194.00675 49.10375) (width 0.2) (layer "F.Cu") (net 1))
 (segment (start 193.9375 53.8875) (end 193.12 53.07) (width 0.2) (layer "F.Cu") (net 1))
 (segment (start 193.12 57.31375) (end 193.12 53.07) (width 0.2) (layer "F.Cu") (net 1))
 (segment (start 194.00675 49.10375) (end 193.12 48.217) (width 0.2) (layer "F.Cu") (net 1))
 (segment (start 192.0915 47.1885) (end 190.02375 47.1885) (width 0.2) (layer "F.Cu") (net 1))
 (segment (start 123.825 73.81875) (end 123.9535 73.94725) (width 0.2) (layer "F.Cu") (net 1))
 (segment (start 180.18125 73.1535) (end 180.975 73.94725) (width 0.2) (layer "F.Cu") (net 1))
 (segment (start 142.08125 66.51625) (end 142.08125 73.1535) (width 0.2) (layer "F.Cu") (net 1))
 (segment (start 180.18125 66.51625) (end 179.33972 66.51625) (width 0.2) (layer "F.Cu") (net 1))
 (segment (start 180.18125 47.46625) (end 182.40375 45.24375) (width 0.2) (layer "F.Cu") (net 1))
 (segment (start 205.70406 48.6655) (end 205.08 48.6655) (width 0.2) (layer "F.Cu") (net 1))
 (segment (start 201.9336 43.8465) (end 191.3961 43.8465) (width 0.2) (layer "F.Cu") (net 1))
 (segment (start 203.192 45.1049) (end 201.9336 43.8465) (width 0.2) (layer "F.Cu") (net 1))
 (segment (start 161.925 73.94725) (end 180.975 73.94725) (width 0.2) (layer "F.Cu") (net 1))
 (segment (start 188.55975 45.7245) (end 190.02375 47.1885) (width 0.2) (layer "F.Cu") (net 1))
 (segment (start 142.08125 47.46625) (end 144.30375 45.24375) (width 0.2) (layer "F.Cu") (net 1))
 (segment (start 180.18125 66.51625) (end 180.18125 73.1535) (width 0.2) (layer "F.Cu") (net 1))
 (segment (start 182.40375 45.24375) (end 184.3485 47.1885) (width 0.2) (layer "F.Cu") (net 1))
 (segment (start 161.13125 47.46625) (end 163.35375 45.24375) (width 0.2) (layer "F.Cu") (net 1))
 (segment (start 123.03125 73.025) (end 123.825 73.81875) (width 0.2) (layer "F.Cu") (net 1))
 (segment (start 190.6986 43.149) (end 189.0739 43.149) (width 0.2) (layer "F.Cu") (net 1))
 (segment (start 142.08125 66.51625) (end 141.23972 66.51625) (width 0.2) (layer "F.Cu") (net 1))
 (segment (start 192.0915 47.1885) (end 193.12 48.217) (width 0.2) (layer "F.Cu") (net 1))
 (segment (start 191.3961 43.8465) (end 190.6986 43.149) (width 0.2) (layer "F.Cu") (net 1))
 (segment (start 123.03125 47.46625) (end 125.25375 45.24375) (width 0.2) (layer "F.Cu") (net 1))
 (segment (start 194.45625 58.65) (end 193.12 57.31375) (width 0.2) (layer "F.Cu") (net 1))
 (segment (start 203.59275 67.02775) (end 206.32675 64.29375) (width 0.2) (layer "F.Cu") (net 1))
 (segment (start 161.13125 66.51625) (end 160.346434 66.51625) (width 0.2) (layer "F.Cu") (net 1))
 (segment (start 144.30375 45.24375) (end 163.35375 45.24375) (width 0.2) (layer "F.Cu") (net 1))
 (segment (start 206.32675 64.29375) (end 206.32675 49.28819) (width 0.2) (layer "F.Cu") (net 1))
 (segment (start 193.12 53.07) (end 193.12 48.217) (width 0.2) (layer "F.Cu") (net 1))
 (segment (start 161.13125 66.51625) (end 161.13125 73.1535) (width 0.2) (layer "F.Cu") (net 1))
 (segment (start 163.35375 45.24375) (end 182.40375 45.24375) (width 0.2) (layer "F.Cu") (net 1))
 (segment (start 142.875 73.94725) (end 161.925 73.94725) (width 0.2) (layer "F.Cu") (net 1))
 (segment (start 189.24 43.55) (end 190.5325 43.55) (width 0.2) (layer "F.Cu") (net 18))
 (segment (start 201.7675 44.2475) (end 202.791 45.271) (width 0.2) (layer "F.Cu") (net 18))
 (segment (start 191.23 44.2475) (end 201.7675 44.2475) (width 0.2) (layer "F.Cu") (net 18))
 (segment (start 188.96075 43.82925) (end 189.24 43.55) (width 0.2) (layer "F.Cu") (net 18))
 (segment (start 195.25625 47.60375) (end 193.364 45.7115) (width 0.2) (layer "F.Cu") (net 18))
 (segment (start 193.364 45.7115) (end 189.58344 45.7115) (width 0.2) (layer "F.Cu") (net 18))
 (segment (start 202.791 45.271) (end 202.791 48.49) (width 0.2) (layer "F.Cu") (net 18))
 (segment (start 204.0295 49.7285) (end 205.26375 49.7285) (width 0.2) (layer "F.Cu") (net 18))
 (segment (start 202.791 48.49) (end 204.0295 49.7285) (width 0.2) (layer "F.Cu") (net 18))
 (segment (start 189.58344 45.7115) (end 188.96075 45.08881) (width 0.2) (layer "F.Cu") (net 18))
 (segment (start 188.96075 45.08881) (end 188.96075 43.82925) (width 0.2) (layer "F.Cu") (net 18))
 (segment (start 190.5325 43.55) (end 191.23 44.2475) (width 0.2) (layer "F.Cu") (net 18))
 (segment (start 200.45625 57.15) (end 201.5 57.15) (width 0.2) (layer "F.Cu") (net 14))
 (segment (start 202.39 45.46) (end 201.5785 44.6485) (width 0.2) (layer "F.Cu") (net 14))
 (segment (start 201.5525 52.3875) (end 202.39 51.55) (width 0.2) (layer "F.Cu") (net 14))
 (segment (start 202.39 51.55) (end 202.39 46.49) (width 0.2) (layer "F.Cu") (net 14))
 (segment (start 202.39 56.26) (end 202.39 51.55) (width 0.2) (layer "F.Cu") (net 14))
 (segment (start 200.45625 47.60375) (end 201.27625 47.60375) (width 0.2) (layer "F.Cu") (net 14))
 (segment (start 202.39 46.49) (end 202.39 45.46) (width 0.2) (layer "F.Cu") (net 14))
 (segment (start 201.5785 44.6485) (end 190.02375 44.6485) (width 0.2) (layer "F.Cu") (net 14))
 (segment (start 201.5 57.15) (end 202.39 56.26) (width 0.2) (layer "F.Cu") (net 14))
 (segment (start 200.4625 52.3875) (end 201.5525 52.3875) (width 0.2) (layer "F.Cu") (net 14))
 (segment (start 201.27625 47.60375) (end 202.39 46.49) (width 0.2) (layer "F.Cu") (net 14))
 (segment (start 196.09 55.6) (end 199.87 55.6) (width 0.2) (layer "F.Cu") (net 16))
 (segment (start 195.28 56.41) (end 196.09 55.6) (width 0.2) (layer "F.Cu") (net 16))
 (segment (start 195.25625 57.15) (end 195.28 57.12625) (width 0.2) (layer "F.Cu") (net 16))
 (segment (start 195.28 57.12625) (end 195.28 56.41) (width 0.2) (layer "F.Cu") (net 16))
 (segment (start 199.87 55.6) (end 200.4625 55.0075) (width 0.2) (layer "F.Cu") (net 16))
 (segment (start 200.4625 55.0075) (end 200.4625 53.8875) (width 0.2) (layer "F.Cu") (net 16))
 (segment (start 178.19275 64.69475) (end 193.224 64.69475) (width 0.2) (layer "F.Cu") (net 6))
 (segment (start 199.92229 64.29375) (end 204.32754 59.8885) (width 0.2) (layer "F.Cu") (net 6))
 (segment (start 173.83125 69.05625) (end 178.19275 64.69475) (width 0.2) (layer "F.Cu") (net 6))
 (segment (start 193.224 64.69475) (end 193.625 64.29375) (width 0.2) (layer "F.Cu") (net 6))
 (segment (start 193.625 64.29375) (end 199.92229 64.29375) (width 0.2) (layer "F.Cu") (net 6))
 (segment (start 204.32754 59.8885) (end 205.26375 59.8885) (width 0.2) (layer "F.Cu") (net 6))
 (segment (start 207.16875 46.5535) (end 205.26375 44.6485) (width 0.2) (layer "F.Cu") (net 11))
 (segment (start 204.89375 73.9375) (end 207.16875 71.6625) (width 0.2) (layer "F.Cu") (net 11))
 (segment (start 207.16875 71.6625) (end 207.16875 46.5535) (width 0.2) (layer "F.Cu") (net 11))
 (segment (start 205.26375 47.1885) (end 205.26375 47.65809) (width 0.2) (layer "F.Cu") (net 10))
 (segment (start 206.72775 67.1035) (end 204.89375 68.9375) (width 0.2) (layer "F.Cu") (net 10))
 (segment (start 206.72775 49.12209) (end 206.72775 67.1035) (width 0.2) (layer "F.Cu") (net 10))
 (segment (start 205.26375 47.65809) (end 206.72775 49.12209) (width 0.2) (layer "F.Cu") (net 10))
 (segment (start 187.8352 57.69995) (end 187.8352 57.43355) (width 0.2) (layer "F.Cu") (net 5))
 (segment (start 187.8352 57.43355) (end 186.5019 56.10025) (width 0.2) (layer "F.Cu") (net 5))
 (segment (start 120.394 56.10025) (end 116.68125 52.3875) (width 0.2) (layer "F.Cu") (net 5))
 (segment (start 190.02375 59.8885) (end 187.8352 57.69995) (width 0.2) (layer "F.Cu") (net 5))
 (segment (start 186.5019 56.10025) (end 120.394 56.10025) (width 0.2) (layer "F.Cu") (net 5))
 (segment (start 116.68125 52.3875) (end 116.68125 50.00625) (width 0.2) (layer "F.Cu") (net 5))
 (segment (start 190.02375 57.3485) (end 188.31725 57.3485) (width 0.2) (layer "F.Cu") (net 3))
 (segment (start 135.73125 52.3875) (end 135.73125 50.00625) (width 0.2) (layer "F.Cu") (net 3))
 (segment (start 139.043 55.69925) (end 135.73125 52.3875) (width 0.2) (layer "F.Cu") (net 3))
 (segment (start 188.31725 57.3485) (end 186.668 55.69925) (width 0.2) (layer "F.Cu") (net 3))
 (segment (start 186.668 55.69925) (end 139.043 55.69925) (width 0.2) (layer "F.Cu") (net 3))
 (segment (start 157.10478 55.29825) (end 189.534 55.29825) (width 0.2) (layer "F.Cu") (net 9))
 (segment (start 154.78125 50.00625) (end 154.78125 52.97472) (width 0.2) (layer "F.Cu") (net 9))
 (segment (start 189.534 55.29825) (end 190.02375 54.8085) (width 0.2) (layer "F.Cu") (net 9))
 (segment (start 154.78125 52.97472) (end 157.10478 55.29825) (width 0.2) (layer "F.Cu") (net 9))
 (segment (start 187.395 54.89725) (end 190.02375 52.2685) (width 0.2) (layer "F.Cu") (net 8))
 (segment (start 173.83125 50.00625) (end 173.83125 52.3875) (width 0.2) (layer "F.Cu") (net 8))
 (segment (start 173.83125 52.3875) (end 176.341 54.89725) (width 0.2) (layer "F.Cu") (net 8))
 (segment (start 176.341 54.89725) (end 187.395 54.89725) (width 0.2) (layer "F.Cu") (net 8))
 (segment (start 139.92665 64.29375) (end 140.32765 63.89275) (width 0.2) (layer "F.Cu") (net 4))
 (segment (start 203.768045 58.746695) (end 203.768045 53.764205) (width 0.2) (layer "F.Cu") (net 4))
 (segment (start 116.68125 69.05625) (end 121.44375 64.29375) (width 0.2) (layer "F.Cu") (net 4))
 (segment (start 140.32765 63.89275) (end 157.1625 63.89275) (width 0.2) (layer "F.Cu") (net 4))
 (segment (start 157.1625 63.89275) (end 157.5635 63.49175) (width 0.2) (layer "F.Cu") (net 4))
 (segment (start 192.71515 63.49175) (end 193.11615 63.09075) (width 0.2) (layer "F.Cu") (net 4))
 (segment (start 121.44375 64.29375) (end 139.92665 64.29375) (width 0.2) (layer "F.Cu") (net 4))
 (segment (start 203.768045 53.764205) (end 205.26375 52.2685) (width 0.2) (layer "F.Cu") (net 4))
 (segment (start 193.11615 63.09075) (end 199.42399 63.09075) (width 0.2) (layer "F.Cu") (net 4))
 (segment (start 157.5635 63.49175) (end 192.71515 63.49175) (width 0.2) (layer "F.Cu") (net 4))
 (segment (start 199.42399 63.09075) (end 203.768045 58.746695) (width 0.2) (layer "F.Cu") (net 4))
 (segment (start 199.59009 63.49175) (end 204.169045 58.912795) (width 0.2) (layer "F.Cu") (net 7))
 (segment (start 159.37765 63.89275) (end 192.88125 63.89275) (width 0.2) (layer "F.Cu") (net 7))
 (segment (start 192.88125 63.89275) (end 193.28225 63.49175) (width 0.2) (layer "F.Cu") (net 7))
 (segment (start 135.73125 69.05625) (end 140.49375 64.29375) (width 0.2) (layer "F.Cu") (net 7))
 (segment (start 204.169045 58.912795) (end 204.169045 55.903205) (width 0.2) (layer "F.Cu") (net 7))
 (segment (start 204.169045 55.903205) (end 205.26375 54.8085) (width 0.2) (layer "F.Cu") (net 7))
 (segment (start 158.97665 64.29375) (end 159.37765 63.89275) (width 0.2) (layer "F.Cu") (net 7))
 (segment (start 193.28225 63.49175) (end 199.59009 63.49175) (width 0.2) (layer "F.Cu") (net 7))
 (segment (start 140.49375 64.29375) (end 158.97665 64.29375) (width 0.2) (layer "F.Cu") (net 7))
 (segment (start 199.75619 63.89275) (end 205.26375 58.38519) (width 0.2) (layer "F.Cu") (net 2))
 (segment (start 159.54375 64.29375) (end 193.04735 64.29375) (width 0.2) (layer "F.Cu") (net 2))
 (segment (start 154.78125 69.05625) (end 159.54375 64.29375) (width 0.2) (layer "F.Cu") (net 2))
 (segment (start 193.44835 63.89275) (end 199.75619 63.89275) (width 0.2) (layer "F.Cu") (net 2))
 (segment (start 193.04735 64.29375) (end 193.44835 63.89275) (width 0.2) (layer "F.Cu") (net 2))
 (segment (start 205.26375 58.38519) (end 205.26375 57.3485) (width 0.2) (layer "F.Cu") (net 2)))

